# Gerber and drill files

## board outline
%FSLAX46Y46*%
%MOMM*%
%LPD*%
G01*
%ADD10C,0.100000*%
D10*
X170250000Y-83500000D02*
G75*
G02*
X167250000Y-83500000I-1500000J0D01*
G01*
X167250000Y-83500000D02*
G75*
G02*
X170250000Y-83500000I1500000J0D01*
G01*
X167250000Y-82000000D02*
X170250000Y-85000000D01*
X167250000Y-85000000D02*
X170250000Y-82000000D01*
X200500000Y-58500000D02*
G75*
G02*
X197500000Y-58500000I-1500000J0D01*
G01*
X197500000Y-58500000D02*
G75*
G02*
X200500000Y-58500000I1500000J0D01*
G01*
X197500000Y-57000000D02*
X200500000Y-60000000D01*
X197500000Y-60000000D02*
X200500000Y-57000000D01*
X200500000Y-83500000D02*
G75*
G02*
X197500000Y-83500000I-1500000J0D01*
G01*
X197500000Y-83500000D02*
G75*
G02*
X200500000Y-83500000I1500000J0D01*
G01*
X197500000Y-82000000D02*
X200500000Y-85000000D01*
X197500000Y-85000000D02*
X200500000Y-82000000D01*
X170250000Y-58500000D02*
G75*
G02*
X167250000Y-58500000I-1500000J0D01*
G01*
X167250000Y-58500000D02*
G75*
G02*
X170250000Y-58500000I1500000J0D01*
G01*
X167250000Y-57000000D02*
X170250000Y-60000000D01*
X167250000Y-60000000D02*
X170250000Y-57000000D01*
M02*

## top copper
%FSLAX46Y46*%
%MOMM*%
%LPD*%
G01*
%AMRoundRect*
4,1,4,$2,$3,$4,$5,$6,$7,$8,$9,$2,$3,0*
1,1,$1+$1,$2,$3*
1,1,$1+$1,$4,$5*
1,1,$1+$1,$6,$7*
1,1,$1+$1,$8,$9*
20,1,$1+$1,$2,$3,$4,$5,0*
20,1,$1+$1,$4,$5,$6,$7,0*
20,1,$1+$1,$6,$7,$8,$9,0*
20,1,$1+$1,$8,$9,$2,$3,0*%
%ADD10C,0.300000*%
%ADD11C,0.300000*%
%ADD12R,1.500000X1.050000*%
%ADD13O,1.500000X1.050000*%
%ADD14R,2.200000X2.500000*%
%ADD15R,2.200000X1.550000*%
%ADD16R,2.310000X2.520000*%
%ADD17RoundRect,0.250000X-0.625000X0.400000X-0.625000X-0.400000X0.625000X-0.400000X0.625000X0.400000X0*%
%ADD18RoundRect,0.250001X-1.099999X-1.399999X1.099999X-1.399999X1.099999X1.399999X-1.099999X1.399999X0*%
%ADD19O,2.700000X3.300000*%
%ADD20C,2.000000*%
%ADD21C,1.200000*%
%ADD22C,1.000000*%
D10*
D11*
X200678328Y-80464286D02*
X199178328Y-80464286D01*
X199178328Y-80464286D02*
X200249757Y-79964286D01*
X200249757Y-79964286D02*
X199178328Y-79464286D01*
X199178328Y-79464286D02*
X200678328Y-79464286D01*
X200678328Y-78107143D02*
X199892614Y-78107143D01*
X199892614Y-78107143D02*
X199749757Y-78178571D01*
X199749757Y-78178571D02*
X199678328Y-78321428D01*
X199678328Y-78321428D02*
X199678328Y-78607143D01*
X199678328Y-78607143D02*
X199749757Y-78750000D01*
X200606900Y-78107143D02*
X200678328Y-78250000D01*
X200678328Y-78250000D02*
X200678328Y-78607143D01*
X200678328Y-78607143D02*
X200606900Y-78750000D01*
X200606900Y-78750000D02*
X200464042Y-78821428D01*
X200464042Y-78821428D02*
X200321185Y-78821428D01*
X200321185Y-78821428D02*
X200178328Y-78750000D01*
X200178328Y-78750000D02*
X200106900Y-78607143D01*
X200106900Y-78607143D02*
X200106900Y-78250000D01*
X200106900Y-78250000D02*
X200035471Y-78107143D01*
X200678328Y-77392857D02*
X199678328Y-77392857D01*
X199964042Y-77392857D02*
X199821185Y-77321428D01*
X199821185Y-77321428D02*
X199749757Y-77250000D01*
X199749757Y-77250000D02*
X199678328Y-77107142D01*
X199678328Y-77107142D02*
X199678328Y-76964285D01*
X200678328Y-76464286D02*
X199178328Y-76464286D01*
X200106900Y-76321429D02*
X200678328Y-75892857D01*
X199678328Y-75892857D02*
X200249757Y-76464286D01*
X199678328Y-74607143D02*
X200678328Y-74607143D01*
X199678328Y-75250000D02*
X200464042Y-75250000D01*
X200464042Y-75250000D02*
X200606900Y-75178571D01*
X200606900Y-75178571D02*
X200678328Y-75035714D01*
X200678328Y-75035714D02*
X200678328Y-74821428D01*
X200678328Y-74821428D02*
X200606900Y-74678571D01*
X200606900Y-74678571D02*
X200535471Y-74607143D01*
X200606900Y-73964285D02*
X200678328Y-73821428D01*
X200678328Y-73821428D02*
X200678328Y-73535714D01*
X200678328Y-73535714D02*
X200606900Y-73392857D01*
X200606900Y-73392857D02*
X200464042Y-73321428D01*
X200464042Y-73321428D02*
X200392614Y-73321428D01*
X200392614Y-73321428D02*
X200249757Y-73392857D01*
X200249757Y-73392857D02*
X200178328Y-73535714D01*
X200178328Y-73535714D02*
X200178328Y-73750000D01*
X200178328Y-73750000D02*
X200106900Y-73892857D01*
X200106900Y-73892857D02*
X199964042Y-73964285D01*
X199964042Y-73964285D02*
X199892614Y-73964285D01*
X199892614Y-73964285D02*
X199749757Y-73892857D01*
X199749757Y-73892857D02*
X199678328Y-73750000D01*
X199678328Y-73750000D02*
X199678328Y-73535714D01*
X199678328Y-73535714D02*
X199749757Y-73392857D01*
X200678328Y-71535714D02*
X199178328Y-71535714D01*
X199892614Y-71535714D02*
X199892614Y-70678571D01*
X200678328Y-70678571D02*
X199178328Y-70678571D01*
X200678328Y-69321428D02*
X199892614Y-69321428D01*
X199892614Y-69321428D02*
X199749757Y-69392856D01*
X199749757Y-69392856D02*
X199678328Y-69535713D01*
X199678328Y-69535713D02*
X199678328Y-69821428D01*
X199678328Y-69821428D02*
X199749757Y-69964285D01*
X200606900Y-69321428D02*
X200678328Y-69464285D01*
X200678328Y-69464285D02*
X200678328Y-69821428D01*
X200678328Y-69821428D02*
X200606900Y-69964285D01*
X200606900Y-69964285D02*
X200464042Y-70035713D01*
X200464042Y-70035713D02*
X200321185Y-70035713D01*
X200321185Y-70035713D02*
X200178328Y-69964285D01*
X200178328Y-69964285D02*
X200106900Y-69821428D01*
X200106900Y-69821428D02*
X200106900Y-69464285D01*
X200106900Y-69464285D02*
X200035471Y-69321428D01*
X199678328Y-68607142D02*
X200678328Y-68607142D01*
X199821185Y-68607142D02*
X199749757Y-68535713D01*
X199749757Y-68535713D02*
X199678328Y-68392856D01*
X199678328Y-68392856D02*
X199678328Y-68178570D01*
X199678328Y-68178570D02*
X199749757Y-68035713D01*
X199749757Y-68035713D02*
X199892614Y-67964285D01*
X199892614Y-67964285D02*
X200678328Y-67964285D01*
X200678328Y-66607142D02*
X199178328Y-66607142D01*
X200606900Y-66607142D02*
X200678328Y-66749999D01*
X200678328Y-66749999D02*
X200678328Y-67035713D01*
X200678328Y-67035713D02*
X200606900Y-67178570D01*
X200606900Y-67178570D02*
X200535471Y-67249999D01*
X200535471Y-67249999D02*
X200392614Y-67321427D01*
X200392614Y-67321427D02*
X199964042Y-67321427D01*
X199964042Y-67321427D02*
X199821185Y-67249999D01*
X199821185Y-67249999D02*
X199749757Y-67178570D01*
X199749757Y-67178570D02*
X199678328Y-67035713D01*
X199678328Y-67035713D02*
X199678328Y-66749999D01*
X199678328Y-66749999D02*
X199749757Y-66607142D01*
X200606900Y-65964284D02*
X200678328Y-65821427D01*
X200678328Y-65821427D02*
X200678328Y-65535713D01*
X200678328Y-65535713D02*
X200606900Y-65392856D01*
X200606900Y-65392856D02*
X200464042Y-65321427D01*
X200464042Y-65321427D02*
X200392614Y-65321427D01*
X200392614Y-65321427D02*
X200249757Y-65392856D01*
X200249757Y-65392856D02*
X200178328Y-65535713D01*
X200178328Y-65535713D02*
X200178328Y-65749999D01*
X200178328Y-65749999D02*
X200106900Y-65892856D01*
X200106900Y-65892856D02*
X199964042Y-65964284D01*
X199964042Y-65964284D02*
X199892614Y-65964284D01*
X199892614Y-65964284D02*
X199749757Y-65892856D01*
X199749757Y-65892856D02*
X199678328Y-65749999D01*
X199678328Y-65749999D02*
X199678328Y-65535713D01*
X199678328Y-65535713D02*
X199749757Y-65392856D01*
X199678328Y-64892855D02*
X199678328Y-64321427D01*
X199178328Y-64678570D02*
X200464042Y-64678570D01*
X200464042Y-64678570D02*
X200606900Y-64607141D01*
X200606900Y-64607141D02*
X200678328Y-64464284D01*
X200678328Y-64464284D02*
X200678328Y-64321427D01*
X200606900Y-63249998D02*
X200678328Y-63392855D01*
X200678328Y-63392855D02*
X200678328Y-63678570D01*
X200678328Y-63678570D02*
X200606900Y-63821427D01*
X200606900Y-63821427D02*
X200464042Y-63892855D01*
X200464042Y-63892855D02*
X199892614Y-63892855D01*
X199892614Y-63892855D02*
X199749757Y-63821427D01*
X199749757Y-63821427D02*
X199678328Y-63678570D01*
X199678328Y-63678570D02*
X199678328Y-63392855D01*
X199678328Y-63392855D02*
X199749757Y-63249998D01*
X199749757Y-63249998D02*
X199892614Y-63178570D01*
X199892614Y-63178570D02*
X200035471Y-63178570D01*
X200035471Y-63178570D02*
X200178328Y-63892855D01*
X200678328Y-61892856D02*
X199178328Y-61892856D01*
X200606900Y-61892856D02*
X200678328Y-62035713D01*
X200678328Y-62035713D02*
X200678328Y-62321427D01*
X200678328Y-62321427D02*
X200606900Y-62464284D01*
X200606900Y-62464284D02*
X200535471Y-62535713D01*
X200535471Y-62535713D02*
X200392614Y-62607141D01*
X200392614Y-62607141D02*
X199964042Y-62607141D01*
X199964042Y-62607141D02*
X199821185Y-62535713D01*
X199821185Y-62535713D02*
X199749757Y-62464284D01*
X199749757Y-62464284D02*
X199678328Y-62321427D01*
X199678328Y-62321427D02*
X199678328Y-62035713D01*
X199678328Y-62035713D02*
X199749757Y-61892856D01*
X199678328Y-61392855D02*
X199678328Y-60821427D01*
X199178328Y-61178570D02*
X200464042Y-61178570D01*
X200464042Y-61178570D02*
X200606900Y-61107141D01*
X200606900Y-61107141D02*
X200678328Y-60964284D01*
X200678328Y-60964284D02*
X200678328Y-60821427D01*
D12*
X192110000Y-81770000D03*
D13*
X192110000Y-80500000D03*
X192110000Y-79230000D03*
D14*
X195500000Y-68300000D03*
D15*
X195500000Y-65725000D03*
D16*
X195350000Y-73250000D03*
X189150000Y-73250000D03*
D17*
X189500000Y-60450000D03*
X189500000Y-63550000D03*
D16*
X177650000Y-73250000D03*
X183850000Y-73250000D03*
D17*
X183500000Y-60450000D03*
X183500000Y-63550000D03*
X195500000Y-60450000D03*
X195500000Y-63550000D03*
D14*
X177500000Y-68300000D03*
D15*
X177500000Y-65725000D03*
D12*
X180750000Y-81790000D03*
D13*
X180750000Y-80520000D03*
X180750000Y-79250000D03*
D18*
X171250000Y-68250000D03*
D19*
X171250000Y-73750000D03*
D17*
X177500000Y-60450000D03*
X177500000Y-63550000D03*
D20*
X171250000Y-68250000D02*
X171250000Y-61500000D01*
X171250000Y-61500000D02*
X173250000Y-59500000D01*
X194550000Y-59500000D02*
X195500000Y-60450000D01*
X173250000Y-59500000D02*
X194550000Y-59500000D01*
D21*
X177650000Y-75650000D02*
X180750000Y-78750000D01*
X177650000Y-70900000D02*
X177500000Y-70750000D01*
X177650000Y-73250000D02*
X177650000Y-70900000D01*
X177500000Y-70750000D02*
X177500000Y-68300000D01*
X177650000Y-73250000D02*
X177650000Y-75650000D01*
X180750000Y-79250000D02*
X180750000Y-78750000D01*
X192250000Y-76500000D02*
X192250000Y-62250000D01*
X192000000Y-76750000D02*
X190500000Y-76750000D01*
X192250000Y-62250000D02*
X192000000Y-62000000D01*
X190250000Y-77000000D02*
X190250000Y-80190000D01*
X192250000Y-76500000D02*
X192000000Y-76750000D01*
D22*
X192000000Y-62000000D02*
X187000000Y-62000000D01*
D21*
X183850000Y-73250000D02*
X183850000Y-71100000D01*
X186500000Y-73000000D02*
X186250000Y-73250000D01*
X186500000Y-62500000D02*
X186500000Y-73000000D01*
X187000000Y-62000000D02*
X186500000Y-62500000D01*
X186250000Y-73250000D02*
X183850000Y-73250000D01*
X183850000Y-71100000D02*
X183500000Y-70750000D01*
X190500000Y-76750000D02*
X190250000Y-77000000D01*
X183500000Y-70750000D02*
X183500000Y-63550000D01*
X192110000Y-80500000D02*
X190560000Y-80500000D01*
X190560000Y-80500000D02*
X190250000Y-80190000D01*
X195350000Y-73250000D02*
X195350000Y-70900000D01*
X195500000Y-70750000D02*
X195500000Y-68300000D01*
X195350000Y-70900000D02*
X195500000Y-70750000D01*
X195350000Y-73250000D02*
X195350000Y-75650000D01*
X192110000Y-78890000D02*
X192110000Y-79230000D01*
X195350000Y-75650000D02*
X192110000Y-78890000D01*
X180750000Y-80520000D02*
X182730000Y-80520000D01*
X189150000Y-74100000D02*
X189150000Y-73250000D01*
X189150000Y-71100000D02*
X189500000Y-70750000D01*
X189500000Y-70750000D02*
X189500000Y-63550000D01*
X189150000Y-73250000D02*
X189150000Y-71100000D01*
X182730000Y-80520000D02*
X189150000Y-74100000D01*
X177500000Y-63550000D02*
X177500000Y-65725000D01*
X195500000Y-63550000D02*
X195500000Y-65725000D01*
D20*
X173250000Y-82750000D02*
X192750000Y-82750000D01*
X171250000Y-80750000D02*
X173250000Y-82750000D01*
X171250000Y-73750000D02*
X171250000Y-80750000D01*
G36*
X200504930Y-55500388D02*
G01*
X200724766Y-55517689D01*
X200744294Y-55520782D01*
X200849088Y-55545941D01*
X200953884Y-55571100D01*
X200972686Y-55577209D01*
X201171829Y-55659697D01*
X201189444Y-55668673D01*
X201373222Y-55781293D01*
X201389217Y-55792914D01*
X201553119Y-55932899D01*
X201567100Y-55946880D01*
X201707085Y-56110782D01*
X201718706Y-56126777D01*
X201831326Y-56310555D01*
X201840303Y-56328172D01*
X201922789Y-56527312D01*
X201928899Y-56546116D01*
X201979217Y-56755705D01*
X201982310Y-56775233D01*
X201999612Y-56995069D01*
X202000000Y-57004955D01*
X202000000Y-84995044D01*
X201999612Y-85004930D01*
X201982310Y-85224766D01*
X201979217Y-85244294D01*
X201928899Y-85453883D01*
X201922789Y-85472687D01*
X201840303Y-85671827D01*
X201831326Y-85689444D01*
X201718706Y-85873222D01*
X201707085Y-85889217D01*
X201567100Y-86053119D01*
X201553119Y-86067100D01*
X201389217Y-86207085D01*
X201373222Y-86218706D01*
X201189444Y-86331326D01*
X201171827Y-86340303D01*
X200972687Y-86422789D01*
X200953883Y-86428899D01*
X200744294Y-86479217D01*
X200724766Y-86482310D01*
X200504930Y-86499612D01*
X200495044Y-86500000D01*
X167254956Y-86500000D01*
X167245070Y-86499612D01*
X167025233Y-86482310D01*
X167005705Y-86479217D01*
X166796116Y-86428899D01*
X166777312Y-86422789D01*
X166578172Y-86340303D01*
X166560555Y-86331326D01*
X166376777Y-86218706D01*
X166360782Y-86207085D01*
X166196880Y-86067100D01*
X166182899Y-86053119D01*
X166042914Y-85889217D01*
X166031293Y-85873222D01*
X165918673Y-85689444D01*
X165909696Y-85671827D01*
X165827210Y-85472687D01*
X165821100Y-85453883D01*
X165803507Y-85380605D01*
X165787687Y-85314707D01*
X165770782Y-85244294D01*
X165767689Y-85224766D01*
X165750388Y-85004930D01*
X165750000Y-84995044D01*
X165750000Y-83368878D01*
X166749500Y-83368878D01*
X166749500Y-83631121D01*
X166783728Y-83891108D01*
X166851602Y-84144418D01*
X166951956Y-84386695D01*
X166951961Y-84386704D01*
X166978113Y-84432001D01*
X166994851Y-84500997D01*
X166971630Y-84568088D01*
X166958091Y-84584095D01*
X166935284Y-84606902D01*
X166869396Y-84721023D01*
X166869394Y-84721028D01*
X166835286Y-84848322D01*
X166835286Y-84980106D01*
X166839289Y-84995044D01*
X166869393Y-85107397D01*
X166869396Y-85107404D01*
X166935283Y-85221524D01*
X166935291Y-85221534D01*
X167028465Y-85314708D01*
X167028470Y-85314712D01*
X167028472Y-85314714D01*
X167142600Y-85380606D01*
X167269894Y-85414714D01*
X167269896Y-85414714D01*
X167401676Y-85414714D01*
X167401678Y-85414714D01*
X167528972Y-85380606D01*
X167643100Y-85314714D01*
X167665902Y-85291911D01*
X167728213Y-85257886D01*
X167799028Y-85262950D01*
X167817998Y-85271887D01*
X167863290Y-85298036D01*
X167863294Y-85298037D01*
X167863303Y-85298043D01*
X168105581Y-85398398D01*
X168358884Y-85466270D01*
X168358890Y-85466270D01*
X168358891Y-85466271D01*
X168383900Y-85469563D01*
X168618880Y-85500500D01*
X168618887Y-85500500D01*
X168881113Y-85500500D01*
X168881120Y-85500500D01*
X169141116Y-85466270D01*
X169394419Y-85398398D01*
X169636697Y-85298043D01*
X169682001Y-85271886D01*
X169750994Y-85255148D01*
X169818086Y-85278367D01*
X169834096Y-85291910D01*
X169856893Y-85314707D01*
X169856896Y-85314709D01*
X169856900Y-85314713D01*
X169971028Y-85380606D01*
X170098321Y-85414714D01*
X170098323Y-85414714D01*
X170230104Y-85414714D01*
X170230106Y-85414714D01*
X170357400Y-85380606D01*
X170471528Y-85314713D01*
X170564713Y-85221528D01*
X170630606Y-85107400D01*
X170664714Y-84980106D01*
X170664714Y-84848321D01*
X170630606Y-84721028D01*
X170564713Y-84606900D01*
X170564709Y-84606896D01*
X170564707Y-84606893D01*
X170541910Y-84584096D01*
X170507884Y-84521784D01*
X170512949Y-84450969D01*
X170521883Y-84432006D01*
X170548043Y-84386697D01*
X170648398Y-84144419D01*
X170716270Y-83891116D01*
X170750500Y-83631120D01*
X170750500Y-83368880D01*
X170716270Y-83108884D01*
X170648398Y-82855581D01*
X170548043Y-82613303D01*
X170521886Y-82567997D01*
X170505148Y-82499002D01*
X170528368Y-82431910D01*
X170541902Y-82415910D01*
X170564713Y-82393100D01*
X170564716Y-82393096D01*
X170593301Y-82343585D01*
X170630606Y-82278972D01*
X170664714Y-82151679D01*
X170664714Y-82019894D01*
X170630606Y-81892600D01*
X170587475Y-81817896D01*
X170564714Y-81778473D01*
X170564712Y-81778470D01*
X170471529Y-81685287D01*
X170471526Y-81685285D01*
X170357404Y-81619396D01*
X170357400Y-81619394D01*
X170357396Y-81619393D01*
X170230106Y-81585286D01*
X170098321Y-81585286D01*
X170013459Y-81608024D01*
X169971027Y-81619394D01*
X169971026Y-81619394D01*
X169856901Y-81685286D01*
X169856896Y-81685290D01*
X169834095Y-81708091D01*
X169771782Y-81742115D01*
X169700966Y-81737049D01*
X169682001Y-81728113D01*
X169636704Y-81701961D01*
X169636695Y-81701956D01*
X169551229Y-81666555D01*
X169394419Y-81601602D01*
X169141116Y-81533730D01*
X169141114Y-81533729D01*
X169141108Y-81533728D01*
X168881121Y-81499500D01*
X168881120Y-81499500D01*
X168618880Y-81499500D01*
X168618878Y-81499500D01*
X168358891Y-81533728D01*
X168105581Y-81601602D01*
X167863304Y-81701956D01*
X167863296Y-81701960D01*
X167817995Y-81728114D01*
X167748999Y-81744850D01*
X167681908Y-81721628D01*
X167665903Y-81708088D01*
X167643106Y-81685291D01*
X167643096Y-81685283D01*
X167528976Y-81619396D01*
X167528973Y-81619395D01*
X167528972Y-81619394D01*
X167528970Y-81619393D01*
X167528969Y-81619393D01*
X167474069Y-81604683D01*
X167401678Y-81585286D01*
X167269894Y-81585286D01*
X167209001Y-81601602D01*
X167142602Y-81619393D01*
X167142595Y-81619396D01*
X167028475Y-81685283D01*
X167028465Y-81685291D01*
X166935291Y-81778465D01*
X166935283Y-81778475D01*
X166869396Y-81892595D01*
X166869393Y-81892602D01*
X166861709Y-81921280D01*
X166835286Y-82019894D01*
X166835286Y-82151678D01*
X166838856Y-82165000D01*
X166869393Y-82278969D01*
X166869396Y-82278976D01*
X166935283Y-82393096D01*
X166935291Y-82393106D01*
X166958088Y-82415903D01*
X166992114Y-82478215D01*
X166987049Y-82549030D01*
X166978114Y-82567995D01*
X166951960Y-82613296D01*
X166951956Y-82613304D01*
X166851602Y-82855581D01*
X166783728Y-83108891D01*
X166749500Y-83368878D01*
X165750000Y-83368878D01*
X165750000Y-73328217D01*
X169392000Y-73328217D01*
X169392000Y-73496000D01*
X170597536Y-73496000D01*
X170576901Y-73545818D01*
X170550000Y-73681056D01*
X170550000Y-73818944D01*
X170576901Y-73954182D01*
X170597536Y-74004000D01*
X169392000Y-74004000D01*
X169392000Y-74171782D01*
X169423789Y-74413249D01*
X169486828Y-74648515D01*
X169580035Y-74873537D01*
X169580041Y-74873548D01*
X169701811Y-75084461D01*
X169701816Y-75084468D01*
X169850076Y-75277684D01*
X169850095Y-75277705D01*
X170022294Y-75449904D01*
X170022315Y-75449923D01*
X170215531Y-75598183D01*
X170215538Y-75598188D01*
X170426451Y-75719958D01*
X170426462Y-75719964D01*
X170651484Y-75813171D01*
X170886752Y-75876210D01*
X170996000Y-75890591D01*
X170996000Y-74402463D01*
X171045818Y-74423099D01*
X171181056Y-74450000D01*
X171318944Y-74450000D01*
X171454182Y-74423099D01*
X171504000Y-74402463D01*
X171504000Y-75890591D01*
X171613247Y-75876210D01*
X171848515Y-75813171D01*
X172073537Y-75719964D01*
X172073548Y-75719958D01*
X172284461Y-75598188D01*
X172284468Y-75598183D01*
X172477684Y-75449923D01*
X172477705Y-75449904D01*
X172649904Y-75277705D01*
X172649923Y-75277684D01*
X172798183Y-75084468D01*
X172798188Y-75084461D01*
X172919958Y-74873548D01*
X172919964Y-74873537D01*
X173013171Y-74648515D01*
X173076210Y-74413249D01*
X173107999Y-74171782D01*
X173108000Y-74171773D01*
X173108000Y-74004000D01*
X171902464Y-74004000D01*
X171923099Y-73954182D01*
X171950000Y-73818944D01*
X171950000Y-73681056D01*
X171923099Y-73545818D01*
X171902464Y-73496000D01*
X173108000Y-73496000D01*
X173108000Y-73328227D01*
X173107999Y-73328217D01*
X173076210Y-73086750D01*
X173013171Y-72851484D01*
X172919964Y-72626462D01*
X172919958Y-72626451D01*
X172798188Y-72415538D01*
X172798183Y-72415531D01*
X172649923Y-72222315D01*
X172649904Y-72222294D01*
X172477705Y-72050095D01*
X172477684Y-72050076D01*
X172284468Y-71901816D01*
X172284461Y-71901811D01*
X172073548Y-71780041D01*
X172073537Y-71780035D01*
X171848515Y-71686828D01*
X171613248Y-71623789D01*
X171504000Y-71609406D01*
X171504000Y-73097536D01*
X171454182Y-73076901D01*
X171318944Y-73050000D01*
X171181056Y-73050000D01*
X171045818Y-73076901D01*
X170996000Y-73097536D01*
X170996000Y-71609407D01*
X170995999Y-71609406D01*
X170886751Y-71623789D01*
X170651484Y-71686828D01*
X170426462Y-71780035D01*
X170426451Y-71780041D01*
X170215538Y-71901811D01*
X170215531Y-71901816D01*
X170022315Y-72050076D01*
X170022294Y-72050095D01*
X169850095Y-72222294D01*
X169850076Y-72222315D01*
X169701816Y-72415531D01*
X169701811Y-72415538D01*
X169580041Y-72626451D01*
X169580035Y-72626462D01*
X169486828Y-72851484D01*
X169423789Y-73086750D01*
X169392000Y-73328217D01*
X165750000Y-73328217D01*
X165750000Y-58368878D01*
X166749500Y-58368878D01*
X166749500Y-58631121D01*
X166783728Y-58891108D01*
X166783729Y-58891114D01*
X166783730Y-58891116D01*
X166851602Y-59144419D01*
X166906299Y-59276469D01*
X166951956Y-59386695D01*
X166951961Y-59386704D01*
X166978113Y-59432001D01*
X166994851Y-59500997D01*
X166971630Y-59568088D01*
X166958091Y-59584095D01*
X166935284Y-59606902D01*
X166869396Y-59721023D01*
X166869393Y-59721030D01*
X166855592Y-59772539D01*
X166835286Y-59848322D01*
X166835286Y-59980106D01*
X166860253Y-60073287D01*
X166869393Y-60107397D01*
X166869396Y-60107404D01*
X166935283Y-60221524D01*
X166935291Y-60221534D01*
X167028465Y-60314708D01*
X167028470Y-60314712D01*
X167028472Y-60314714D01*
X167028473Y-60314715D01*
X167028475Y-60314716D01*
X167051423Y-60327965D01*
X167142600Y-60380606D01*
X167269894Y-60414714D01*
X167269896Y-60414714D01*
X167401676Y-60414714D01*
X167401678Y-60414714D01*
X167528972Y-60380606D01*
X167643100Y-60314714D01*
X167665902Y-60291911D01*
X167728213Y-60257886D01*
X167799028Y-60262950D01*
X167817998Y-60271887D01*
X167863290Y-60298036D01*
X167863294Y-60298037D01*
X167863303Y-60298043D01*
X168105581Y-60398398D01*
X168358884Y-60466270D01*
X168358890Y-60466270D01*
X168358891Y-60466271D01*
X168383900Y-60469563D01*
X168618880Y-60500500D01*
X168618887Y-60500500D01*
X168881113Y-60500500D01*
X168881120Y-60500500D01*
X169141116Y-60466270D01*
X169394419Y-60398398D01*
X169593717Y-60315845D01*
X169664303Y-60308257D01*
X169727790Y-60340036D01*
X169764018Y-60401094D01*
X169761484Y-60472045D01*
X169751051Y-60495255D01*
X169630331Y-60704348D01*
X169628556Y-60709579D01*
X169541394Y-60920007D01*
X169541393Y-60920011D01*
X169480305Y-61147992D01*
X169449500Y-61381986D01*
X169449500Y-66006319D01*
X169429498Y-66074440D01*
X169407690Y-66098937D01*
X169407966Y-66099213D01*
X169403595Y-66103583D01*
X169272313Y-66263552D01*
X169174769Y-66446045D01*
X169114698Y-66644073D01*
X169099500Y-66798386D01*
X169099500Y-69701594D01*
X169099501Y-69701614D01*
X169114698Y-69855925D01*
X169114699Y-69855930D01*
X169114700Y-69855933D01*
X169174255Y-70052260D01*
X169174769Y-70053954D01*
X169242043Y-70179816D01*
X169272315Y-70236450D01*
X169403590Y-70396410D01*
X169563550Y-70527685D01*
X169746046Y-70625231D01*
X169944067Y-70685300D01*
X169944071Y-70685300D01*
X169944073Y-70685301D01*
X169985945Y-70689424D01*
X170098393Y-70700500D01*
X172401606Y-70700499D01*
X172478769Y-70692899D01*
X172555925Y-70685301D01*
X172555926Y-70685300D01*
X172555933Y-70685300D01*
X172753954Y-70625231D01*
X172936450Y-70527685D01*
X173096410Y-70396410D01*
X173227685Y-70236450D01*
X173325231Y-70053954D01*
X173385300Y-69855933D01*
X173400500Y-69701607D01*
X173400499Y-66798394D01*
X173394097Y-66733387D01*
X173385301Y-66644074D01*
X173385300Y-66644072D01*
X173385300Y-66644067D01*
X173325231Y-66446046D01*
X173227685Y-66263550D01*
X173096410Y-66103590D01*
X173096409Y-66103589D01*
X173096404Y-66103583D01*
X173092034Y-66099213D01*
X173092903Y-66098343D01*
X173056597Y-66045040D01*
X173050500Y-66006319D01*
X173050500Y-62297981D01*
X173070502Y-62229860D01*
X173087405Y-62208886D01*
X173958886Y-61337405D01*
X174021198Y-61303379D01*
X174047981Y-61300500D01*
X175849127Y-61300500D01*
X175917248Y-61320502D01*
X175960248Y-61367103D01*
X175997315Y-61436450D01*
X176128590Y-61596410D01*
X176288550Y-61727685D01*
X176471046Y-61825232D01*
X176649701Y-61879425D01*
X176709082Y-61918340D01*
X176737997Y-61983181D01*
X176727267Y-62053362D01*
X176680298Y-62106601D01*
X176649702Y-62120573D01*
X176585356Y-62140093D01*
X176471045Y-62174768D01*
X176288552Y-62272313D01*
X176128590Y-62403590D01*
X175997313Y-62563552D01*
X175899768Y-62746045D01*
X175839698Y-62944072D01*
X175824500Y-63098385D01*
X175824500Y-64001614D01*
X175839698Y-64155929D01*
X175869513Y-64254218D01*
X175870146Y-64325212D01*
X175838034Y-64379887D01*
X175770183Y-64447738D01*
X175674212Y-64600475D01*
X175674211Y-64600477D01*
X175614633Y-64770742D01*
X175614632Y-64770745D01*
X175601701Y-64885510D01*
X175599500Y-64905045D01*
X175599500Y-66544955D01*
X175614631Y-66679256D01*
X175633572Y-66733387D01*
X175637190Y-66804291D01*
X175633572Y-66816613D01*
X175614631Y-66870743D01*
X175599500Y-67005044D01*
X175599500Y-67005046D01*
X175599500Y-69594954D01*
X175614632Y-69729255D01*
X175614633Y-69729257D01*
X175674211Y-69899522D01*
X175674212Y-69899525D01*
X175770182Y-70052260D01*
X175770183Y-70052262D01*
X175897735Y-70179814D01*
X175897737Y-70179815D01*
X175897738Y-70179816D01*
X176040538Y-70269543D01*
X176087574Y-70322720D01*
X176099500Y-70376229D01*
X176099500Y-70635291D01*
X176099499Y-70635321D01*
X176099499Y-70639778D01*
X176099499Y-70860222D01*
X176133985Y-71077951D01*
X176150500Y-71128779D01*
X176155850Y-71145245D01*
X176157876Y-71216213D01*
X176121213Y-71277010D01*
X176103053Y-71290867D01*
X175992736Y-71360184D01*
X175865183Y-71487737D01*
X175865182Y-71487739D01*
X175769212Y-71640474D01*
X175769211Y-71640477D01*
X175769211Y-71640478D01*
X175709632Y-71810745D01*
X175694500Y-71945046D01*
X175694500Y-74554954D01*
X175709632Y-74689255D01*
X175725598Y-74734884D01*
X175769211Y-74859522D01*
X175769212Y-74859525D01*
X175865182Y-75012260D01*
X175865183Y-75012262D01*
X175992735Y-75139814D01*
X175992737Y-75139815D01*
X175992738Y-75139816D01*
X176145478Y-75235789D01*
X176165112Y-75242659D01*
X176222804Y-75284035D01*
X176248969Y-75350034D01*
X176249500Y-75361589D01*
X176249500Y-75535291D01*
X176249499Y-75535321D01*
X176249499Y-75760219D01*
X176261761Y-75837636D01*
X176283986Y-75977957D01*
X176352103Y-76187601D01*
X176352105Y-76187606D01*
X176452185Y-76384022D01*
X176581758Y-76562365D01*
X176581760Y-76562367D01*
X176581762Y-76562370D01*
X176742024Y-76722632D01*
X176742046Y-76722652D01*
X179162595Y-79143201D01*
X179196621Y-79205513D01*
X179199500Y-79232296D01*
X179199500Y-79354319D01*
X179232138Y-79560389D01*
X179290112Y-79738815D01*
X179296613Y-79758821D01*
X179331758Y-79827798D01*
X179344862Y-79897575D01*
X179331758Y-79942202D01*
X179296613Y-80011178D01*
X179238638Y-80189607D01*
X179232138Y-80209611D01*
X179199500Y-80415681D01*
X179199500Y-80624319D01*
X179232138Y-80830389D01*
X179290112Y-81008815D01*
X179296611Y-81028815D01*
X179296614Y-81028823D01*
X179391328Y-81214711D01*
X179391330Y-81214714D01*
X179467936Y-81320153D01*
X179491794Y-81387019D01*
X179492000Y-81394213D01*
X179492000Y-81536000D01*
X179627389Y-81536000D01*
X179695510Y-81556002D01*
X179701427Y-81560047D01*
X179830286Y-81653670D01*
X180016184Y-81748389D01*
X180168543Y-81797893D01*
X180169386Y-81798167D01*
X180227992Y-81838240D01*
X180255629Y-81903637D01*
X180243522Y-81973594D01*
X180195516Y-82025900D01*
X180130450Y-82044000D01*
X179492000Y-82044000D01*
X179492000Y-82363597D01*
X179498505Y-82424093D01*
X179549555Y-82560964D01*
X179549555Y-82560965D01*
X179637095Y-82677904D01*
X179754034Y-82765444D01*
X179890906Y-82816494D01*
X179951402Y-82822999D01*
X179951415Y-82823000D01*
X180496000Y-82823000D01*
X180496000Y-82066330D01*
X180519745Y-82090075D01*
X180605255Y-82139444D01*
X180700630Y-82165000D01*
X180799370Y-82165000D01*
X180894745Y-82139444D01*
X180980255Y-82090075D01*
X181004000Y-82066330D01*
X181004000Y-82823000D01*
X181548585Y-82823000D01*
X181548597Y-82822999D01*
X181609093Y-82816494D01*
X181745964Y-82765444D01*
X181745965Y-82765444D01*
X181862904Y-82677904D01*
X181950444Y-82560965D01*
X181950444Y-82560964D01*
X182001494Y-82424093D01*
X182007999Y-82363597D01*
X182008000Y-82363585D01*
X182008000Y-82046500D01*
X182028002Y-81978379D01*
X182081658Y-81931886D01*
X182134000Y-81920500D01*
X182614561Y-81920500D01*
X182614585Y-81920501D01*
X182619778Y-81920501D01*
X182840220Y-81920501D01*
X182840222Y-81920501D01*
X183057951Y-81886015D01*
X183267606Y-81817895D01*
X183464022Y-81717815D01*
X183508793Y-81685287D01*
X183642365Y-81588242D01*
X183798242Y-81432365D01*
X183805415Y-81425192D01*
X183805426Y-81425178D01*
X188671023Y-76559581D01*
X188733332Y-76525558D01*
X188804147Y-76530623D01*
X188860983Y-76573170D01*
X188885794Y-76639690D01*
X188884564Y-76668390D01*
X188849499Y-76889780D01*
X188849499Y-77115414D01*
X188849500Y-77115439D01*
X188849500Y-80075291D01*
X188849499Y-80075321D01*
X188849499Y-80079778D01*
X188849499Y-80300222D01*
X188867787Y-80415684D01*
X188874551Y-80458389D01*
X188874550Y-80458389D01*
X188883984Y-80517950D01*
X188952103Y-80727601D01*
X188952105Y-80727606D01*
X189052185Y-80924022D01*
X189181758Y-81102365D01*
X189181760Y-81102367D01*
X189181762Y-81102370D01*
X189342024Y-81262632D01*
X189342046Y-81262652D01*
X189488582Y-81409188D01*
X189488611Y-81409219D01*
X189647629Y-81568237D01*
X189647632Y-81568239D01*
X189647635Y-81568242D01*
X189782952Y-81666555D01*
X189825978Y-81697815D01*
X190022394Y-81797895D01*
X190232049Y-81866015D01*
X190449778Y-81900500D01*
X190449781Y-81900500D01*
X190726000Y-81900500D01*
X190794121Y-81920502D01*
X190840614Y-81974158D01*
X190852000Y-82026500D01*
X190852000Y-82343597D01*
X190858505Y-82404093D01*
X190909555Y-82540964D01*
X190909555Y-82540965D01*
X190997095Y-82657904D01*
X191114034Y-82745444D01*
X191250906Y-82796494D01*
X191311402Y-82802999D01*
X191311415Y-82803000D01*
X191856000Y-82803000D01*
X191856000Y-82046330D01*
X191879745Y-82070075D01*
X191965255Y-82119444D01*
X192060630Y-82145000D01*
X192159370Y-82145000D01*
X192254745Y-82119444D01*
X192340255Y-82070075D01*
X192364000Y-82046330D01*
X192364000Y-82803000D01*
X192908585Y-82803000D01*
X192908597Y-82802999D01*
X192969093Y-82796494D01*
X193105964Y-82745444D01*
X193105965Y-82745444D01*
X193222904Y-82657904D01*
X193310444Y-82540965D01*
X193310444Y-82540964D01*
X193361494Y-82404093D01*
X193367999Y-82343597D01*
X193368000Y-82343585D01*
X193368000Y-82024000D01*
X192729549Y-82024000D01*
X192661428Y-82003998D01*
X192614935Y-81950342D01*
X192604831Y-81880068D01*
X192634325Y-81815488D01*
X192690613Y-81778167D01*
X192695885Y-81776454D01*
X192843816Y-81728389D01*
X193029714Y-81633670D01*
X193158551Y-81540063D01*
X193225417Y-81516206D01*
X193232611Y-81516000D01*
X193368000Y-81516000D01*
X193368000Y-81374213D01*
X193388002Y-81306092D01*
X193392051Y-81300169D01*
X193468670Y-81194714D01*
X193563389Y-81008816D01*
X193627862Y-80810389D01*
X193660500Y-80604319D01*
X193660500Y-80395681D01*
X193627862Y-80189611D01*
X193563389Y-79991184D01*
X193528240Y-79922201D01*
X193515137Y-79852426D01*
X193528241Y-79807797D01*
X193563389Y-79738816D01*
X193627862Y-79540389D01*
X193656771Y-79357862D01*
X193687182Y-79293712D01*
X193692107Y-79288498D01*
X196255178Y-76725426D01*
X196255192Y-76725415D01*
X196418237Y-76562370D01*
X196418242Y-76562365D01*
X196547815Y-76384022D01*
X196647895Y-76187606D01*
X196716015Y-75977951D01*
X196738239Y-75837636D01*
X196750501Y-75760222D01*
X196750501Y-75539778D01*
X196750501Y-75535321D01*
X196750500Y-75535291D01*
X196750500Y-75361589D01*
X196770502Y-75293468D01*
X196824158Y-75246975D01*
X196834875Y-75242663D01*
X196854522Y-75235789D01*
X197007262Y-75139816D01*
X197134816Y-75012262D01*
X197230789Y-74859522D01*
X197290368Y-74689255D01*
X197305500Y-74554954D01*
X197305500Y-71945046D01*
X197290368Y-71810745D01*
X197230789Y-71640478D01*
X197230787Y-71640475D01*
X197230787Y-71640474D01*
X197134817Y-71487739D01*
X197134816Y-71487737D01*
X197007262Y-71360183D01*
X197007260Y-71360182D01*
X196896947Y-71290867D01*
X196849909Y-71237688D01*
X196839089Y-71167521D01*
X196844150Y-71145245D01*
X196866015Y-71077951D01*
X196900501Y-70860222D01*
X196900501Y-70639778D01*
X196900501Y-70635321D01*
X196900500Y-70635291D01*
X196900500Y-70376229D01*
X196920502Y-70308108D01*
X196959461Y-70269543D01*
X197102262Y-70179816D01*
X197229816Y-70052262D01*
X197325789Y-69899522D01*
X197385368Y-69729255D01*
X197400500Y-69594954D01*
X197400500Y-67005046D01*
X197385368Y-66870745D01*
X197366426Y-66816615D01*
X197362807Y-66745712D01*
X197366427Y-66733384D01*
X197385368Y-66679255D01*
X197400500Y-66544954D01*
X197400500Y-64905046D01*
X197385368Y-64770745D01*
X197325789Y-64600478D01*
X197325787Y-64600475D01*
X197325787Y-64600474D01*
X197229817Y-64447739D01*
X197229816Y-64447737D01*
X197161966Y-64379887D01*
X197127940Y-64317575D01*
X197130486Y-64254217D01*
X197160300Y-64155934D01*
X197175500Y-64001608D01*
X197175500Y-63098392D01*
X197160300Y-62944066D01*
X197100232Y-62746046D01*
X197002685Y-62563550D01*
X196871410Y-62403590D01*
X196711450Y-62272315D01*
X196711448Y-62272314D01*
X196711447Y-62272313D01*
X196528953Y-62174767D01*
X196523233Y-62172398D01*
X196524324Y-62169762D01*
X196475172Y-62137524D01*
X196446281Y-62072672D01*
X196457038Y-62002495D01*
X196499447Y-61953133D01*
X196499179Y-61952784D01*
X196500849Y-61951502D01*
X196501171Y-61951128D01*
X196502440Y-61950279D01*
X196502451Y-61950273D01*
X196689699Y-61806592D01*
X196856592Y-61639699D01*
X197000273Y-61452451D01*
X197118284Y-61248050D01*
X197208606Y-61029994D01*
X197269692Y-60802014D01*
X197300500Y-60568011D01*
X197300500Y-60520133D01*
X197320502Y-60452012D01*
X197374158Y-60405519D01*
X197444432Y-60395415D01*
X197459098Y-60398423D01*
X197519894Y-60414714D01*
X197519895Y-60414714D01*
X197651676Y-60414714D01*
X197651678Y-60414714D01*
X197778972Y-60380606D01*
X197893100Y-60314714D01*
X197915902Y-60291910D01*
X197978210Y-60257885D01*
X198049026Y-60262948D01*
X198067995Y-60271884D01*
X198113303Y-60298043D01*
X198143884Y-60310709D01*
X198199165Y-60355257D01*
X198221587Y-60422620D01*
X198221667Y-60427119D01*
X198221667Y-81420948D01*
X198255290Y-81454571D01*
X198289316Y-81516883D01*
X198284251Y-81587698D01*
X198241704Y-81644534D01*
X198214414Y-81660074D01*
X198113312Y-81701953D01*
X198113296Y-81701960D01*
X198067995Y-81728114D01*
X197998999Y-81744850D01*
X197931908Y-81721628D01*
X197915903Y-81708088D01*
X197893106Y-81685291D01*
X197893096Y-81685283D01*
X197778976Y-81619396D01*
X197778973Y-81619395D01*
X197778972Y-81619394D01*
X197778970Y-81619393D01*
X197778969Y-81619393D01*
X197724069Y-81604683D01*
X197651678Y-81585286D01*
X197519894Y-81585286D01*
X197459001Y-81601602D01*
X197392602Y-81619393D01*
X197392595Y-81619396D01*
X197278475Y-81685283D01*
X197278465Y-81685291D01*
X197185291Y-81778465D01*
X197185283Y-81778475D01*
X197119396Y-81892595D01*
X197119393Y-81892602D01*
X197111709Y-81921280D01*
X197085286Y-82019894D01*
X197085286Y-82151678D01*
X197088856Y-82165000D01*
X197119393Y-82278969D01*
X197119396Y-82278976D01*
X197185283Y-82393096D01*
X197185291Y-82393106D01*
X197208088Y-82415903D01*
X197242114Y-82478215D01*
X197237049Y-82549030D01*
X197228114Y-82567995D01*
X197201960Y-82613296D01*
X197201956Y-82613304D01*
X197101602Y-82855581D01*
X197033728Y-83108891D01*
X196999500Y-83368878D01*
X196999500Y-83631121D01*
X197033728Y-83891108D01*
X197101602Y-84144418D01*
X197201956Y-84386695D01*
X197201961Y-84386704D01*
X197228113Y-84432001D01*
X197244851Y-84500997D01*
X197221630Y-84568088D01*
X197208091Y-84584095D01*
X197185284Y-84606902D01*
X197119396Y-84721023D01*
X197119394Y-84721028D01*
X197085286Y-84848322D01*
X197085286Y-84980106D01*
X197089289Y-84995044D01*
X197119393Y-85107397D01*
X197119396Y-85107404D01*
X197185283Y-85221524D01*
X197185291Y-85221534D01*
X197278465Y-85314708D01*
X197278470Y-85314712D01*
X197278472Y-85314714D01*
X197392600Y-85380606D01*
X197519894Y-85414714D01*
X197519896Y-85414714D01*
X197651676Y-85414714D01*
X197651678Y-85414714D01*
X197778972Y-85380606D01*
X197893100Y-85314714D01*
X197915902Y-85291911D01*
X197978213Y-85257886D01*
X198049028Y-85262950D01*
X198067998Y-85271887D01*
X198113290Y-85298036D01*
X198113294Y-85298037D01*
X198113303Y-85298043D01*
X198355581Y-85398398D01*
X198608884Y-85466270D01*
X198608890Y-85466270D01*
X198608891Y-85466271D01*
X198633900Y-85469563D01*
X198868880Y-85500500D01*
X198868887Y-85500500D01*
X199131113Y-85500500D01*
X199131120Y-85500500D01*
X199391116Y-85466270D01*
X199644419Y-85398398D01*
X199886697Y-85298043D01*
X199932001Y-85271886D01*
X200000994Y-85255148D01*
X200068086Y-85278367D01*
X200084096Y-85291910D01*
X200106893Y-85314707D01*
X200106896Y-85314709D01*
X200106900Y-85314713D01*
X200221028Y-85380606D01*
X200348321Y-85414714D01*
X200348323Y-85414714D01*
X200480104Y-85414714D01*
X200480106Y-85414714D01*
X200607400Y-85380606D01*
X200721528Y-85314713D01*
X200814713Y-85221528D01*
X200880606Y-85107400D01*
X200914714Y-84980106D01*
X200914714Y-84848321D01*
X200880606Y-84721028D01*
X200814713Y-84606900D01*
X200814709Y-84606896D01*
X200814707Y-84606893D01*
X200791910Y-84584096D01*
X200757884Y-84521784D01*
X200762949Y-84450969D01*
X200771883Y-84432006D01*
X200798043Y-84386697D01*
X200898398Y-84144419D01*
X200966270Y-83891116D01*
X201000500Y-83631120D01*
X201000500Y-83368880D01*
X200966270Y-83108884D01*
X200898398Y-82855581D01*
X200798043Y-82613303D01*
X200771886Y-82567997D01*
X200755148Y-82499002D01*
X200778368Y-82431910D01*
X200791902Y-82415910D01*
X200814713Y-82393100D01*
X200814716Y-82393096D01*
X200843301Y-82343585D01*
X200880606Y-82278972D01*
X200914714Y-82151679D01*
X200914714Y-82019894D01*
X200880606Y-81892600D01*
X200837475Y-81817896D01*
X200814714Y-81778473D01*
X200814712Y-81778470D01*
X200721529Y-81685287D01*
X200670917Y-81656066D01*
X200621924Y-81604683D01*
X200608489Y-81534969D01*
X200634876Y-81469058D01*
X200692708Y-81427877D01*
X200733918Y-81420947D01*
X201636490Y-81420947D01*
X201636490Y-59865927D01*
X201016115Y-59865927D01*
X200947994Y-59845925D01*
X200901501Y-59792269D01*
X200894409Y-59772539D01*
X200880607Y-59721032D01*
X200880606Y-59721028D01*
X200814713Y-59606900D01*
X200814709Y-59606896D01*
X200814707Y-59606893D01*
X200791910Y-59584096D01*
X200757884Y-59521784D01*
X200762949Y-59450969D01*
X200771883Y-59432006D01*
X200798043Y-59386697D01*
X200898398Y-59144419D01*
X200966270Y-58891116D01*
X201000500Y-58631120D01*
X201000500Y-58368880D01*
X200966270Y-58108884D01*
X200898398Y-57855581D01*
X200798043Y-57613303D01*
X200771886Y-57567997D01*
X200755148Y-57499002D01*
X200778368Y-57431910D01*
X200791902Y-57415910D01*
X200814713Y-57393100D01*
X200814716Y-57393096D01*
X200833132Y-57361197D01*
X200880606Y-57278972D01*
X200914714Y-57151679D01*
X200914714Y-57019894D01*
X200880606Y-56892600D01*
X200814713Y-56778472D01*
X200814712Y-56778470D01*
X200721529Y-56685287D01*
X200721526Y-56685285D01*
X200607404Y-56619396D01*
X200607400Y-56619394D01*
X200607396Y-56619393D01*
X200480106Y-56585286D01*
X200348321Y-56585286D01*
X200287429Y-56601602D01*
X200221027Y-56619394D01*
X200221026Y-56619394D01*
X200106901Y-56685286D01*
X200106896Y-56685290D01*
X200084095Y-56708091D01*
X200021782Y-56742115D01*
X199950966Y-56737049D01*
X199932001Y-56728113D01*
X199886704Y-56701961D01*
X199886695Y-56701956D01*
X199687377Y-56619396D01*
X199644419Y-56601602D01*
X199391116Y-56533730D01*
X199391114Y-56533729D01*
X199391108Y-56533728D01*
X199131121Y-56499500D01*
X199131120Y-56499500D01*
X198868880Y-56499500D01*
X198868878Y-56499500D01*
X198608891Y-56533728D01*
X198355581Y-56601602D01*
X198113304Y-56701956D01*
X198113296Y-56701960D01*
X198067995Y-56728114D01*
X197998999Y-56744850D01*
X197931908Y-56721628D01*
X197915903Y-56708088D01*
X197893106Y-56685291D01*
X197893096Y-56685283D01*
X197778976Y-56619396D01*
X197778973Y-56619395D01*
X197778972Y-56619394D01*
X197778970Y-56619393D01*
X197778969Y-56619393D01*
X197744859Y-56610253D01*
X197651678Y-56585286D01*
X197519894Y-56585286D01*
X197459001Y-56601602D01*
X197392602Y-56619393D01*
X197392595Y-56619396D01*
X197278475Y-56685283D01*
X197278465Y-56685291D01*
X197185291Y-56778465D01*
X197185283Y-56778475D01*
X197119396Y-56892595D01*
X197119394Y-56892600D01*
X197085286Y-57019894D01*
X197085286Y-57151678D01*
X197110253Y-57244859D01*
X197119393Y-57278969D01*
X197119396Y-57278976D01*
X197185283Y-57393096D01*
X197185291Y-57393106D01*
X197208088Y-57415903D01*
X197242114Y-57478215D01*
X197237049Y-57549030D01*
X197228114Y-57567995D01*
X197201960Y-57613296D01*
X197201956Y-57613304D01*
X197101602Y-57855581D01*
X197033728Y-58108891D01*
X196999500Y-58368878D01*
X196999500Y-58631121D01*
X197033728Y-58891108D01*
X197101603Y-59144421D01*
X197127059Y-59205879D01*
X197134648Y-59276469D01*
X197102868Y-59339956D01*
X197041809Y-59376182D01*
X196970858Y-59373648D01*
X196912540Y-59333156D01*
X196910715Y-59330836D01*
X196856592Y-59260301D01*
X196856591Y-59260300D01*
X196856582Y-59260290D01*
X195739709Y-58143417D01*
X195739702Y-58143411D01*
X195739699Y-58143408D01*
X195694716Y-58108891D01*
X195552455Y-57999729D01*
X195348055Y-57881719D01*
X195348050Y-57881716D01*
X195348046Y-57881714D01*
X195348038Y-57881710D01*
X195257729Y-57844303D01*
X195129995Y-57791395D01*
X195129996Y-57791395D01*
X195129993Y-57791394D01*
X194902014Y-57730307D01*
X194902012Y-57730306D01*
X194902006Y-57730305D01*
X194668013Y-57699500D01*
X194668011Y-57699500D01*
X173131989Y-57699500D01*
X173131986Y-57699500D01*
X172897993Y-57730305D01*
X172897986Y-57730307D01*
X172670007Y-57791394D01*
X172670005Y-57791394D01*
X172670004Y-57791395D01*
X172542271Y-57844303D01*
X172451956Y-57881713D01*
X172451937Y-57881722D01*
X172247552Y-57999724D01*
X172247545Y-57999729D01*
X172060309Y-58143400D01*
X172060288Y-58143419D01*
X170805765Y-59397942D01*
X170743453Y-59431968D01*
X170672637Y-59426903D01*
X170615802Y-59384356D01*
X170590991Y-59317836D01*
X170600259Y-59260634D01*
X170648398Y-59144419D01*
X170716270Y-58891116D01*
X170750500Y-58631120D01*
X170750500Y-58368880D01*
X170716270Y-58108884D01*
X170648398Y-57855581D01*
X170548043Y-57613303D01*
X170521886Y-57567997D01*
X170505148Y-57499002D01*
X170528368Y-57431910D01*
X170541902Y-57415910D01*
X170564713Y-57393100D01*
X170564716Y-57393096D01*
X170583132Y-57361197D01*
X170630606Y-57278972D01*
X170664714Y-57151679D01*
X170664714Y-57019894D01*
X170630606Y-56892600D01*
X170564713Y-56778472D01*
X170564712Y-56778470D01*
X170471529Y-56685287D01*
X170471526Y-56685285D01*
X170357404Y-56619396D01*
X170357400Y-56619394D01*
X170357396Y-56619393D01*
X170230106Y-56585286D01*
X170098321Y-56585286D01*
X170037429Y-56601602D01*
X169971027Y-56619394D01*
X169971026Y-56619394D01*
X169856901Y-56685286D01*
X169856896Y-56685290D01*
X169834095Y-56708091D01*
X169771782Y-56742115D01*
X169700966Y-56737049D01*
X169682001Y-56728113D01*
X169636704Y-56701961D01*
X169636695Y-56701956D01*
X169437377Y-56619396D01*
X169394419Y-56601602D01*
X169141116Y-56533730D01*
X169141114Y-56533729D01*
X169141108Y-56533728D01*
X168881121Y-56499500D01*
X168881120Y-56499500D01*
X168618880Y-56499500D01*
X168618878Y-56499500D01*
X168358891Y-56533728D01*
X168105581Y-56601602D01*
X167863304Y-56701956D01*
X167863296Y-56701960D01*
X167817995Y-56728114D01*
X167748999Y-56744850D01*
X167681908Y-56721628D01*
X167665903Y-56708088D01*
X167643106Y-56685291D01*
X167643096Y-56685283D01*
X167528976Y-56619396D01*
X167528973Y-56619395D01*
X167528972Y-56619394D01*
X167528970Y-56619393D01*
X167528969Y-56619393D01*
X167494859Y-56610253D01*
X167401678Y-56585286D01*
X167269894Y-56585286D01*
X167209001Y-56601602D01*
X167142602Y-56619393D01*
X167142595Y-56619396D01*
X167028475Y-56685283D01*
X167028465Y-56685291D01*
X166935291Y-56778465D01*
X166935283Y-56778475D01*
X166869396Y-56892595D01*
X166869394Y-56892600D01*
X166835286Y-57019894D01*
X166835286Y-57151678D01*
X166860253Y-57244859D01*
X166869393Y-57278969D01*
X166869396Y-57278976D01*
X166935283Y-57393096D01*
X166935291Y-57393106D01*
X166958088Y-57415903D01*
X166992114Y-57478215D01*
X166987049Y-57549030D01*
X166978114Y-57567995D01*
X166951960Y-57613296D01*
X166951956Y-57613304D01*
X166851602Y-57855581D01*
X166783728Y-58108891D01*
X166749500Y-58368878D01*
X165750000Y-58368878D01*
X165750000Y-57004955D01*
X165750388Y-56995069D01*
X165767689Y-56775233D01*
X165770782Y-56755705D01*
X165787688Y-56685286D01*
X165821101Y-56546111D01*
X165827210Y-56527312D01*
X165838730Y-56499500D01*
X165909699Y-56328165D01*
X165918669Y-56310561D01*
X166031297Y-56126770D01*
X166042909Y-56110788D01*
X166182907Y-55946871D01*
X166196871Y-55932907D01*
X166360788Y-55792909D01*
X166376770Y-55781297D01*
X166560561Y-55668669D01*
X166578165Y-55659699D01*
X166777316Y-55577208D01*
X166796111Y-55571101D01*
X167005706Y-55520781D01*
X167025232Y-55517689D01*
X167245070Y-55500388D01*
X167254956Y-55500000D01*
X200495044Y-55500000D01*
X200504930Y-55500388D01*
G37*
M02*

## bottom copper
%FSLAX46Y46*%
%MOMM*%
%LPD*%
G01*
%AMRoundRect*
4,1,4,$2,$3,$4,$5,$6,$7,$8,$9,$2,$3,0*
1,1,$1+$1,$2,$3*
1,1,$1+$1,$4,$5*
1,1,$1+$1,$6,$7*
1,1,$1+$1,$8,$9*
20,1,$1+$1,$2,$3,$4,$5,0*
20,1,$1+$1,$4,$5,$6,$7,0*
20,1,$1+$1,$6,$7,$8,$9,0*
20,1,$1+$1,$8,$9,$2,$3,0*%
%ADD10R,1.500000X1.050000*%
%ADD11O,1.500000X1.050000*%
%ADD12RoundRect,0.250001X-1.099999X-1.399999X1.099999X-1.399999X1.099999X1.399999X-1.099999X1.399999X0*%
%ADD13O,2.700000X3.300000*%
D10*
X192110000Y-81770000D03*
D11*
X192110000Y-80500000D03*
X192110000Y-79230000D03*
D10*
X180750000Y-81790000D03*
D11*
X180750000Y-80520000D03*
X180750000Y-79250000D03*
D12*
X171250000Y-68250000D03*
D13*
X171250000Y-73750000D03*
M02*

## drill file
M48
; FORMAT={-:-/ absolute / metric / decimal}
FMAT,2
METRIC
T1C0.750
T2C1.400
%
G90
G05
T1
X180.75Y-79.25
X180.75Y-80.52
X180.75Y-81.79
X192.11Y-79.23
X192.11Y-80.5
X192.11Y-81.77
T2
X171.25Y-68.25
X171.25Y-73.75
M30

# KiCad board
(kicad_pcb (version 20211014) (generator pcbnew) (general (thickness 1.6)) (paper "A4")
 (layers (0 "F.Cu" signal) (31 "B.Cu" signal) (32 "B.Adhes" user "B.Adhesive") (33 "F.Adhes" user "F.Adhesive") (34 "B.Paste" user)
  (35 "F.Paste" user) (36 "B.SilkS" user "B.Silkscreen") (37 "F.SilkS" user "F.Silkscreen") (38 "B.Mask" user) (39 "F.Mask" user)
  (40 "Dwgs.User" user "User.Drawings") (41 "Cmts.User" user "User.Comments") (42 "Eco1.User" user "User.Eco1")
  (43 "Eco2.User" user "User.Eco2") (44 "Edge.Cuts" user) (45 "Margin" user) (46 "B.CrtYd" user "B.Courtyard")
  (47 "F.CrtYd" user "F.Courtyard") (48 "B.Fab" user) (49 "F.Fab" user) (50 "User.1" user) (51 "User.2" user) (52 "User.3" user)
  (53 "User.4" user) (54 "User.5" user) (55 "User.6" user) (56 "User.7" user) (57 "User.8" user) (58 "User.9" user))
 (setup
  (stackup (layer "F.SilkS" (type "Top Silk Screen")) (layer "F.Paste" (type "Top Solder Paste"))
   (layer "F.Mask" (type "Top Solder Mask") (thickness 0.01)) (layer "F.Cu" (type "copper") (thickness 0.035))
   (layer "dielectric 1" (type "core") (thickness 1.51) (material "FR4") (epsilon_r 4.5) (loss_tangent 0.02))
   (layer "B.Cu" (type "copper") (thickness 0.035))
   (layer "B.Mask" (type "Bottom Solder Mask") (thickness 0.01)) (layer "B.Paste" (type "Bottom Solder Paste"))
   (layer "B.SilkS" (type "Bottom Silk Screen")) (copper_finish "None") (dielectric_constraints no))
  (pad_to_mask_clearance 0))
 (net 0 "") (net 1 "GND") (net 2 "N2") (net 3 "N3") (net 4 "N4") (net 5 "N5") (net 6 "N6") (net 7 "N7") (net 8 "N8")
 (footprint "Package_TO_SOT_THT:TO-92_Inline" (layer "F.Cu") (at 192.11 81.77 90)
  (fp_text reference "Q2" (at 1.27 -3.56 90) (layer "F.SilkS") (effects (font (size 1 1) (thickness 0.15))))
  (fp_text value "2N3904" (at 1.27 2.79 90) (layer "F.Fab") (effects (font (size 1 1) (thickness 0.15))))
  (pad "1" thru_hole rect (at 0 0 90) (size 1.05 1.5) (drill 0.75) (layers *.Cu *.Mask) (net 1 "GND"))
  (pad "2" thru_hole oval (at 1.27 0 90) (size 1.05 1.5) (drill 0.75) (layers *.Cu *.Mask) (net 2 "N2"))
  (pad "3" thru_hole oval (at 2.54 0 90) (size 1.05 1.5) (drill 0.75) (layers *.Cu *.Mask) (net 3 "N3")))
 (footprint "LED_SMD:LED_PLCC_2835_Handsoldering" (layer "F.Cu") (at 195.5 67.25 90)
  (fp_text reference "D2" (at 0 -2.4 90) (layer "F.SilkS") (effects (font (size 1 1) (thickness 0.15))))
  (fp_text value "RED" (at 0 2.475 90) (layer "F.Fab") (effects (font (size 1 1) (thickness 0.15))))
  (pad "1" smd rect (at -1.05 0 90) (size 2.5 2.2) (layers "F.Cu" "F.Paste" "F.Mask") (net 3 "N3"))
  (pad "2" smd rect (at 1.525 0 90) (size 1.55 2.2) (layers "F.Cu" "F.Paste" "F.Mask") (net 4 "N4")))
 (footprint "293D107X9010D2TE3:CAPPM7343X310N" (layer "F.Cu") (at 192.25 73.25 180)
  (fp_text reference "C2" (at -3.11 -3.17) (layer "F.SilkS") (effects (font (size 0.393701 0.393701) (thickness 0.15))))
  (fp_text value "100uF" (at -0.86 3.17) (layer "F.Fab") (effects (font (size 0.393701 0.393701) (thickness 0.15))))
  (pad "1" smd rect locked (at -3.1 0 180) (size 2.31 2.52) (layers "F.Cu" "F.Paste" "F.Mask") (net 3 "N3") (solder_mask_margin 0.102))
  (pad "2" smd rect locked (at 3.1 0 180) (size 2.31 2.52) (layers "F.Cu" "F.Paste" "F.Mask") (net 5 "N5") (solder_mask_margin 0.102)))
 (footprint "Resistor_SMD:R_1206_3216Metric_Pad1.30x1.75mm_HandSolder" (layer "F.Cu") (at 189.5 62 -90)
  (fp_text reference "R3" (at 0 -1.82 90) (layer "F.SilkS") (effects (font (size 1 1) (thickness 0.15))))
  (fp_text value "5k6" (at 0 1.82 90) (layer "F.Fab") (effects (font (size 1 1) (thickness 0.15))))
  (pad "1" smd roundrect (at -1.55 0 270) (size 1.3 1.75) (layers "F.Cu" "F.Paste" "F.Mask") (roundrect_rratio 0.192308) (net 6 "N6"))
  (pad "2" smd roundrect (at 1.55 0 270) (size 1.3 1.75) (layers "F.Cu" "F.Paste" "F.Mask") (roundrect_rratio 0.192308) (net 5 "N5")))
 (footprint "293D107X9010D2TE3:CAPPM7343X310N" (layer "F.Cu") (at 180.75 73.25)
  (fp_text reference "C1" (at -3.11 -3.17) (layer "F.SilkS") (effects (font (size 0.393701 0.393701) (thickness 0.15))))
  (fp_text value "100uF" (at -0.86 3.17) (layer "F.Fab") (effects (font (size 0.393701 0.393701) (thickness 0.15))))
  (pad "1" smd rect locked (at -3.1 0) (size 2.31 2.52) (layers "F.Cu" "F.Paste" "F.Mask") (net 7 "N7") (solder_mask_margin 0.102))
  (pad "2" smd rect locked (at 3.1 0) (size 2.31 2.52) (layers "F.Cu" "F.Paste" "F.Mask") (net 2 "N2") (solder_mask_margin 0.102)))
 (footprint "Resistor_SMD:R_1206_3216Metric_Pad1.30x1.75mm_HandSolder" (layer "F.Cu") (at 183.5 62 -90)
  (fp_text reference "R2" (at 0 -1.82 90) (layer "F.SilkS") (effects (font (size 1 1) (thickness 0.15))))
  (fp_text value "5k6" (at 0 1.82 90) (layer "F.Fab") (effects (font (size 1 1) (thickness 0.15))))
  (pad "1" smd roundrect (at -1.55 0 270) (size 1.3 1.75) (layers "F.Cu" "F.Paste" "F.Mask") (roundrect_rratio 0.192308) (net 6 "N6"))
  (pad "2" smd roundrect (at 1.55 0 270) (size 1.3 1.75) (layers "F.Cu" "F.Paste" "F.Mask") (roundrect_rratio 0.192308) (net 2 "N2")))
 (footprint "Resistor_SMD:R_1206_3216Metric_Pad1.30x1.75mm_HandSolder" (layer "F.Cu") (at 195.5 62 -90)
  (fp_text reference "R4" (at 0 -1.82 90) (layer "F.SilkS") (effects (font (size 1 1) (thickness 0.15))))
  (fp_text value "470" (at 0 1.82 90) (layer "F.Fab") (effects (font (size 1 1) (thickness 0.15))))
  (pad "1" smd roundrect (at -1.55 0 270) (size 1.3 1.75) (layers "F.Cu" "F.Paste" "F.Mask") (roundrect_rratio 0.192308) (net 6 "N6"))
  (pad "2" smd roundrect (at 1.55 0 270) (size 1.3 1.75) (layers "F.Cu" "F.Paste" "F.Mask") (roundrect_rratio 0.192308) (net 4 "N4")))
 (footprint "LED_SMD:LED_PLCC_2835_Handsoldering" (layer "F.Cu") (at 177.5 67.25 90)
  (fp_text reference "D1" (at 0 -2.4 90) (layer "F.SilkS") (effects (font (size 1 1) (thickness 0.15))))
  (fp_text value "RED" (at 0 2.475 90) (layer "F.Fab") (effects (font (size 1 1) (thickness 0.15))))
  (pad "1" smd rect (at -1.05 0 90) (size 2.5 2.2) (layers "F.Cu" "F.Paste" "F.Mask") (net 7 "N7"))
  (pad "2" smd rect (at 1.525 0 90) (size 1.55 2.2) (layers "F.Cu" "F.Paste" "F.Mask") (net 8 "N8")))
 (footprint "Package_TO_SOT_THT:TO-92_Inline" (layer "F.Cu") (at 180.75 81.79 90)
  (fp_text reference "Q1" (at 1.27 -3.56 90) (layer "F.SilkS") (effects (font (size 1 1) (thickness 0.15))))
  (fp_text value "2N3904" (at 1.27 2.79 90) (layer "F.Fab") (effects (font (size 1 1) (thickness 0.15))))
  (pad "1" thru_hole rect (at 0 0 90) (size 1.05 1.5) (drill 0.75) (layers *.Cu *.Mask) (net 1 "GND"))
  (pad "2" thru_hole oval (at 1.27 0 90) (size 1.05 1.5) (drill 0.75) (layers *.Cu *.Mask) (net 5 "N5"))
  (pad "3" thru_hole oval (at 2.54 0 90) (size 1.05 1.5) (drill 0.75) (layers *.Cu *.Mask) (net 7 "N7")))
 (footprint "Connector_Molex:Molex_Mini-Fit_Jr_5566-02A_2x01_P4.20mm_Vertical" (layer "F.Cu") (at 171.25 68.25)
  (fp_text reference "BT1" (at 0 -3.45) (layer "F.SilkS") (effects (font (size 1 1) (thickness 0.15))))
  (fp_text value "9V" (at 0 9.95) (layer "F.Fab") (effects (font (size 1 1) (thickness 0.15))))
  (pad "1" thru_hole roundrect (at 0 0) (size 2.7 3.3) (drill 1.4) (layers *.Cu *.Mask) (roundrect_rratio 0.092593) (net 6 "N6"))
  (pad "2" thru_hole oval (at 0 5.5) (size 2.7 3.3) (drill 1.4) (layers *.Cu *.Mask) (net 1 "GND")))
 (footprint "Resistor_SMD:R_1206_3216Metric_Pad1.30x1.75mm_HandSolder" (layer "F.Cu") (at 177.5 62 -90)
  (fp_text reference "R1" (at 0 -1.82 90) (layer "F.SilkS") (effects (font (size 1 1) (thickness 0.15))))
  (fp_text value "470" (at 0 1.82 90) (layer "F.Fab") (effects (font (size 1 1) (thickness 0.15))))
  (pad "1" smd roundrect (at -1.55 0 270) (size 1.3 1.75) (layers "F.Cu" "F.Paste" "F.Mask") (roundrect_rratio 0.192308) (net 6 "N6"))
  (pad "2" smd roundrect (at 1.55 0 270) (size 1.3 1.75) (layers "F.Cu" "F.Paste" "F.Mask") (roundrect_rratio 0.192308) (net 8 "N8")))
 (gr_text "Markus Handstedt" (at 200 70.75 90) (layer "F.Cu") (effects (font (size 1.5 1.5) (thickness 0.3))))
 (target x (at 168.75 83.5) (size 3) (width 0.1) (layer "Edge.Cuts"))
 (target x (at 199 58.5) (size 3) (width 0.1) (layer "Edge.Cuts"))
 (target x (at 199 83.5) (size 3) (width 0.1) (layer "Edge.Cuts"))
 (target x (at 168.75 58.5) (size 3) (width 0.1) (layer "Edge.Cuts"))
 (segment (start 171.25 68.25) (end 171.25 61.5) (width 2) (layer "F.Cu") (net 6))
 (segment (start 171.25 61.5) (end 173.25 59.5) (width 2) (layer "F.Cu") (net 6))
 (segment (start 194.55 59.5) (end 195.5 60.45) (width 2) (layer "F.Cu") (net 6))
 (segment (start 173.25 59.5) (end 194.55 59.5) (width 2) (layer "F.Cu") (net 6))
 (segment (start 177.65 75.65) (end 180.75 78.75) (width 1.2) (layer "F.Cu") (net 7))
 (segment (start 177.65 70.9) (end 177.5 70.75) (width 1.2) (layer "F.Cu") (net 7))
 (segment (start 177.65 73.25) (end 177.65 70.9) (width 1.2) (layer "F.Cu") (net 7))
 (segment (start 177.5 70.75) (end 177.5 68.3) (width 1.2) (layer "F.Cu") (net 7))
 (segment (start 177.65 73.25) (end 177.65 75.65) (width 1.2) (layer "F.Cu") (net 7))
 (segment (start 180.75 79.25) (end 180.75 78.75) (width 1.2) (layer "F.Cu") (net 7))
 (segment (start 192.25 76.5) (end 192.25 62.25) (width 1.2) (layer "F.Cu") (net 2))
 (segment (start 192 76.75) (end 190.5 76.75) (width 1.2) (layer "F.Cu") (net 2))
 (segment (start 192.25 62.25) (end 192 62) (width 1.2) (layer "F.Cu") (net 2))
 (segment (start 190.25 77) (end 190.25 80.19) (width 1.2) (layer "F.Cu") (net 2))
 (segment (start 192.25 76.5) (end 192 76.75) (width 1.2) (layer "F.Cu") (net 2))
 (segment (start 192 62) (end 187 62) (width 1) (layer "F.Cu") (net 2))
 (segment (start 183.85 73.25) (end 183.85 71.1) (width 1.2) (layer "F.Cu") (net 2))
 (segment (start 186.5 73) (end 186.25 73.25) (width 1.2) (layer "F.Cu") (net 2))
 (segment (start 186.5 62.5) (end 186.5 73) (width 1.2) (layer "F.Cu") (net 2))
 (segment (start 187 62) (end 186.5 62.5) (width 1.2) (layer "F.Cu") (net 2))
 (segment (start 186.25 73.25) (end 183.85 73.25) (width 1.2) (layer "F.Cu") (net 2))
 (segment (start 183.85 71.1) (end 183.5 70.75) (width 1.2) (layer "F.Cu") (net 2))
 (segment (start 190.5 76.75) (end 190.25 77) (width 1.2) (layer "F.Cu") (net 2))
 (segment (start 183.5 70.75) (end 183.5 63.55) (width 1.2) (layer "F.Cu") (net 2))
 (segment (start 192.11 80.5) (end 190.56 80.5) (width 1.2) (layer "F.Cu") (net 2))
 (segment (start 190.56 80.5) (end 190.25 80.19) (width 1.2) (layer "F.Cu") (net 2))
 (segment (start 195.35 73.25) (end 195.35 70.9) (width 1.2) (layer "F.Cu") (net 3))
 (segment (start 195.5 70.75) (end 195.5 68.3) (width 1.2) (layer "F.Cu") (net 3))
 (segment (start 195.35 70.9) (end 195.5 70.75) (width 1.2) (layer "F.Cu") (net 3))
 (segment (start 195.35 73.25) (end 195.35 75.65) (width 1.2) (layer "F.Cu") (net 3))
 (segment (start 192.11 78.89) (end 192.11 79.23) (width 1.2) (layer "F.Cu") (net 3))
 (segment (start 195.35 75.65) (end 192.11 78.89) (width 1.2) (layer "F.Cu") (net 3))
 (segment (start 180.75 80.52) (end 182.73 80.52) (width 1.2) (layer "F.Cu") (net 5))
 (segment (start 189.15 74.1) (end 189.15 73.25) (width 1.2) (layer "F.Cu") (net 5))
 (segment (start 189.15 71.1) (end 189.5 70.75) (width 1.2) (layer "F.Cu") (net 5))
 (segment (start 189.5 70.75) (end 189.5 63.55) (width 1.2) (layer "F.Cu") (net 5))
 (segment (start 189.15 73.25) (end 189.15 71.1) (width 1.2) (layer "F.Cu") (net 5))
 (segment (start 182.73 80.52) (end 189.15 74.1) (width 1.2) (layer "F.Cu") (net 5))
 (segment (start 177.5 63.55) (end 177.5 65.725) (width 1.2) (layer "F.Cu") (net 8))
 (segment (start 195.5 63.55) (end 195.5 65.725) (width 1.2) (layer "F.Cu") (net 4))
 (segment (start 173.25 82.75) (end 192.75 82.75) (width 2) (layer "F.Cu") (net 1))
 (segment (start 171.25 80.75) (end 173.25 82.75) (width 2) (layer "F.Cu") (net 1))
 (segment (start 171.25 73.75) (end 171.25 80.75) (width 2) (layer "F.Cu") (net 1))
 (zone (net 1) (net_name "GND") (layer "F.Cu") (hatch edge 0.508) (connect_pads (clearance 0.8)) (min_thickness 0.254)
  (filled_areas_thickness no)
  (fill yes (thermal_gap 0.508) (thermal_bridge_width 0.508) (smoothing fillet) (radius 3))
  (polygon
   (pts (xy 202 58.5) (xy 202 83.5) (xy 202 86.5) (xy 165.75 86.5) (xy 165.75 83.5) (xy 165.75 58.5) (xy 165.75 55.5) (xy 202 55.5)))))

